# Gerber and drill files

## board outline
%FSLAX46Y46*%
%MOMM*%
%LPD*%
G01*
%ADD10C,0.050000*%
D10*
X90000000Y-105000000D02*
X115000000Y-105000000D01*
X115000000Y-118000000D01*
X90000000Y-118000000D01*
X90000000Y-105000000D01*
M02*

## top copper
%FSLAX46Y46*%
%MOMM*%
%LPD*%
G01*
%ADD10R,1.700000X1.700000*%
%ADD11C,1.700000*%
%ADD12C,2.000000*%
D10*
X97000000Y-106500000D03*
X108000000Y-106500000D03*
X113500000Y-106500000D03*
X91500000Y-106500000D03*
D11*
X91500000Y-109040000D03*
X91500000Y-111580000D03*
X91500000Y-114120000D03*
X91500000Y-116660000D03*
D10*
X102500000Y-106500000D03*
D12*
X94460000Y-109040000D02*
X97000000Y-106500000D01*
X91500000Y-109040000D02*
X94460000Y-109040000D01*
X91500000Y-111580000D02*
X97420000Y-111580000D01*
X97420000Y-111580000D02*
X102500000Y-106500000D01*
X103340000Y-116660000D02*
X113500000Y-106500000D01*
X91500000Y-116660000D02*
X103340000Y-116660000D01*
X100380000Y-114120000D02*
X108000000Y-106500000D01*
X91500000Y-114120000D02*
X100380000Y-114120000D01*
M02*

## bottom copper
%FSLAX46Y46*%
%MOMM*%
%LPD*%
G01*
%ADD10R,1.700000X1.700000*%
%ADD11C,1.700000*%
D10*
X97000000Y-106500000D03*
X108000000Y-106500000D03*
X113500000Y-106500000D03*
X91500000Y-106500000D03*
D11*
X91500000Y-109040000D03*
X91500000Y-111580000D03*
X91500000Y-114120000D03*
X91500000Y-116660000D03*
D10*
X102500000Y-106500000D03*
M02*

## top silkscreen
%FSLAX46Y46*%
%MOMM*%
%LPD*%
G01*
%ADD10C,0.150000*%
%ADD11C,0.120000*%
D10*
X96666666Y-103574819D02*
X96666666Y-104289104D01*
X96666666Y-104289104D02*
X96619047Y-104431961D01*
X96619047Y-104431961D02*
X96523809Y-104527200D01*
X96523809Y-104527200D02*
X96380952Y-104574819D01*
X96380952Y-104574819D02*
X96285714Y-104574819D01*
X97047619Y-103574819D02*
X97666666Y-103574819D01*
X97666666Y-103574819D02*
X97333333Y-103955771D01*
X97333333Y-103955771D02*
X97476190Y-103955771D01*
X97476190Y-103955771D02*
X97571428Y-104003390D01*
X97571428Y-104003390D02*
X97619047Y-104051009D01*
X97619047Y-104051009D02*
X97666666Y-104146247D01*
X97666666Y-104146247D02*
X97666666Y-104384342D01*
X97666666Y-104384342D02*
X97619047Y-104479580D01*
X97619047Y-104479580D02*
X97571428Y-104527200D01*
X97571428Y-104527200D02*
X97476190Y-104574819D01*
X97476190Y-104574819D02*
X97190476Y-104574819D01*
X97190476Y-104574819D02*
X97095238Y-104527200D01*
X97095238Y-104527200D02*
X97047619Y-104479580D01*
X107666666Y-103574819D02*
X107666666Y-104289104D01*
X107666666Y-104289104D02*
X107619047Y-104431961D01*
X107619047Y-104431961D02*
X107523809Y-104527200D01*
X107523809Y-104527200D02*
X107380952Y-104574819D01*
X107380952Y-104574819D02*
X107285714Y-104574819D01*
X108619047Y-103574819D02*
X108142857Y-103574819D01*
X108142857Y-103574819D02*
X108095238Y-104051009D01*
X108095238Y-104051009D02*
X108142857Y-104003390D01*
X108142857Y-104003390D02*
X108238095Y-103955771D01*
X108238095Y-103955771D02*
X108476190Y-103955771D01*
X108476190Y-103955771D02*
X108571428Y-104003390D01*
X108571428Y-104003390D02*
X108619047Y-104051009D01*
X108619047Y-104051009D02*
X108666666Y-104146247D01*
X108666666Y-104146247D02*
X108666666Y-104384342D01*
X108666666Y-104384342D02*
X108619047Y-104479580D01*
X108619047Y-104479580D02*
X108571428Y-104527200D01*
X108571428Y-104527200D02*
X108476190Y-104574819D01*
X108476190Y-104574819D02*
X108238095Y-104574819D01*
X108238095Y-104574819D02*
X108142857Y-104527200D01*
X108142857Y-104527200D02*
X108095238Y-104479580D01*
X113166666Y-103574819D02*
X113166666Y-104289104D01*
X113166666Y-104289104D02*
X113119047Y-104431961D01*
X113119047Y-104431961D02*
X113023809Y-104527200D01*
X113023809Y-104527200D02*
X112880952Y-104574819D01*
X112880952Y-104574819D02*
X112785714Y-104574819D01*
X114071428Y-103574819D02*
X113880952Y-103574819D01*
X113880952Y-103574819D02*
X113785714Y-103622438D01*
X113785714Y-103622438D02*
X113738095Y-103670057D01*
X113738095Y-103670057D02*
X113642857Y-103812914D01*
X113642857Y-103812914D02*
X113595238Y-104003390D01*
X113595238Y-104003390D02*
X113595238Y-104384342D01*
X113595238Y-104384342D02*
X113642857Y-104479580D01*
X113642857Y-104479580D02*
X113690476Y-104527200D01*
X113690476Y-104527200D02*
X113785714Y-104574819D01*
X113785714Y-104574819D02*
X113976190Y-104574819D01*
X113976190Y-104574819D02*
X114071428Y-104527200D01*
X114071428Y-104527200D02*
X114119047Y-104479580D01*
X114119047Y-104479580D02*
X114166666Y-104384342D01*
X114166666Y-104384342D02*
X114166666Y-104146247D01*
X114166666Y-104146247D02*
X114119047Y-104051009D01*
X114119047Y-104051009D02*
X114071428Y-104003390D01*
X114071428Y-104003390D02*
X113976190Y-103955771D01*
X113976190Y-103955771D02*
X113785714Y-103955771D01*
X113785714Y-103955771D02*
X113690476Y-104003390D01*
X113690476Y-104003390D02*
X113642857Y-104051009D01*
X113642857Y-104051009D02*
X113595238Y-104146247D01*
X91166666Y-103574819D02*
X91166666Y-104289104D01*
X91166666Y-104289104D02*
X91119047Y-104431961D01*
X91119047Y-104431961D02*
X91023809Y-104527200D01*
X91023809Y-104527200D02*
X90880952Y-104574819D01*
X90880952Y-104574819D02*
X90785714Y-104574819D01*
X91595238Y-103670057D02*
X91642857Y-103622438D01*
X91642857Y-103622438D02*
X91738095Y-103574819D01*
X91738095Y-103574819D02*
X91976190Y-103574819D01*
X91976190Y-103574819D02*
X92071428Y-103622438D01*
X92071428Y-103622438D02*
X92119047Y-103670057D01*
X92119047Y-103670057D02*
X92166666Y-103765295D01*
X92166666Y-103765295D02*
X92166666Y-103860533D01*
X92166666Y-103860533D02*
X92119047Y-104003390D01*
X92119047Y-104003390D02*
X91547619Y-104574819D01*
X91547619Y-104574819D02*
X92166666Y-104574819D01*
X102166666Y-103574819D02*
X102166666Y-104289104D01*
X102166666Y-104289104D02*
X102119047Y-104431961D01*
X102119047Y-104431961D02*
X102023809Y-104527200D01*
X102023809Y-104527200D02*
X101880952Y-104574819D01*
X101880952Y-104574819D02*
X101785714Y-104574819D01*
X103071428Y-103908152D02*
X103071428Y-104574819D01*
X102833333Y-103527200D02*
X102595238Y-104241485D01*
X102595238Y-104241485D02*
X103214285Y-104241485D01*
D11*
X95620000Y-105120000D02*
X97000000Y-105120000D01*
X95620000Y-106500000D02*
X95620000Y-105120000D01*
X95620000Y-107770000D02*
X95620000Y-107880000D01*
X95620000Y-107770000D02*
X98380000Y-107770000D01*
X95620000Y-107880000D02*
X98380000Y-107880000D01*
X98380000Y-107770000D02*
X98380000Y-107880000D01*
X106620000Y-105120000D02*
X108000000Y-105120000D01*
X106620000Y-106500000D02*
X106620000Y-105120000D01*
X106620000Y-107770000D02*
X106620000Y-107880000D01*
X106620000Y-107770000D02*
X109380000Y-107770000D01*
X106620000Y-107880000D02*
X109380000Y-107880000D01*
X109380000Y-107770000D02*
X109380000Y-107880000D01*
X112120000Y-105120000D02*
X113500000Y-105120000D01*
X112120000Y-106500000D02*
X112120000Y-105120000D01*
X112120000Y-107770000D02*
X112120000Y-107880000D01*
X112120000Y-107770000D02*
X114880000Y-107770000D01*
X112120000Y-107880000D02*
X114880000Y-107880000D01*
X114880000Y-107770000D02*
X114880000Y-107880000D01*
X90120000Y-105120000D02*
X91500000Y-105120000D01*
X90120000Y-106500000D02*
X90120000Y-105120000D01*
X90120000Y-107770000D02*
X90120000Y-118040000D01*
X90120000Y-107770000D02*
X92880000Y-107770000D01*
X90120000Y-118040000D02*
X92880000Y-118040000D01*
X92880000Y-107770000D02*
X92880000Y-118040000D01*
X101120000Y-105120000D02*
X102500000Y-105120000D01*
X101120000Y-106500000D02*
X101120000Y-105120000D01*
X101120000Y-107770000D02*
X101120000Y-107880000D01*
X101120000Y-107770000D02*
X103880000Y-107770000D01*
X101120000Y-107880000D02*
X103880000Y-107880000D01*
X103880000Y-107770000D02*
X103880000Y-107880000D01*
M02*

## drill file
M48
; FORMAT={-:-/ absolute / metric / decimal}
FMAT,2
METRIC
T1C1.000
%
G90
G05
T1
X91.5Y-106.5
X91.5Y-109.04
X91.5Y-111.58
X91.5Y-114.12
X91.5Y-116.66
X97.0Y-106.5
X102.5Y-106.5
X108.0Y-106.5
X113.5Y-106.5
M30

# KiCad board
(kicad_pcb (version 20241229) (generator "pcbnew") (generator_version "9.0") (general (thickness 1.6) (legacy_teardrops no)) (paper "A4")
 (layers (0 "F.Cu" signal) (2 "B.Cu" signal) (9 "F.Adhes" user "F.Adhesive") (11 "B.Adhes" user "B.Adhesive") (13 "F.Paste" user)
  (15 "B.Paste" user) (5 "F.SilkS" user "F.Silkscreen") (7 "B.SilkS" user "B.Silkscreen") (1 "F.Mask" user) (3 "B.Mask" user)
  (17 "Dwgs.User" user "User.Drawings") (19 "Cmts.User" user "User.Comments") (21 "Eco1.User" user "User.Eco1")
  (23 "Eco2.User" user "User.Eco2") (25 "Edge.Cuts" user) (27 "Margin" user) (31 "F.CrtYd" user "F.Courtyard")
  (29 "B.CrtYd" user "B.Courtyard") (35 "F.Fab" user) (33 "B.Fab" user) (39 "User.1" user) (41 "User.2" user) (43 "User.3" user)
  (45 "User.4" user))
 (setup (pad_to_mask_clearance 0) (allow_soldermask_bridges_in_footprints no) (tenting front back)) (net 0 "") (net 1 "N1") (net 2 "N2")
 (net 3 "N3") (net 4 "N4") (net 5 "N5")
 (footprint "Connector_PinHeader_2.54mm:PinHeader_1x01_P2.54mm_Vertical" (layer "F.Cu") (at 97 106.5)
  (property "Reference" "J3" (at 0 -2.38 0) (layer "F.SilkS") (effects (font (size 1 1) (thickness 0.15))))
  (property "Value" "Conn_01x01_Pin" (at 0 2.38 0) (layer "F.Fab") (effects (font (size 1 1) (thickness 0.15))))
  (fp_line (start -1.38 -1.38) (end 0 -1.38) (stroke (width 0.12) (type solid)) (layer "F.SilkS"))
  (fp_line (start -1.38 0) (end -1.38 -1.38) (stroke (width 0.12) (type solid)) (layer "F.SilkS"))
  (fp_line (start -1.38 1.27) (end -1.38 1.38) (stroke (width 0.12) (type solid)) (layer "F.SilkS"))
  (fp_line (start -1.38 1.27) (end 1.38 1.27) (stroke (width 0.12) (type solid)) (layer "F.SilkS"))
  (fp_line (start -1.38 1.38) (end 1.38 1.38) (stroke (width 0.12) (type solid)) (layer "F.SilkS"))
  (fp_line (start 1.38 1.27) (end 1.38 1.38) (stroke (width 0.12) (type solid)) (layer "F.SilkS"))
  (pad "1" thru_hole rect (at 0 0) (size 1.7 1.7) (drill 1) (layers "*.Cu" "*.Mask") (remove_unused_layers no) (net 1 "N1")))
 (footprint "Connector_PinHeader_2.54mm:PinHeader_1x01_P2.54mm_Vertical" (layer "F.Cu") (at 108 106.5)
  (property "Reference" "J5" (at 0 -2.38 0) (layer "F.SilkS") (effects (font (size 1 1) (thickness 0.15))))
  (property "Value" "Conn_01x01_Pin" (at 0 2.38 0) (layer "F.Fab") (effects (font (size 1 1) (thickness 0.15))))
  (fp_line (start -1.38 -1.38) (end 0 -1.38) (stroke (width 0.12) (type solid)) (layer "F.SilkS"))
  (fp_line (start -1.38 0) (end -1.38 -1.38) (stroke (width 0.12) (type solid)) (layer "F.SilkS"))
  (fp_line (start -1.38 1.27) (end -1.38 1.38) (stroke (width 0.12) (type solid)) (layer "F.SilkS"))
  (fp_line (start -1.38 1.27) (end 1.38 1.27) (stroke (width 0.12) (type solid)) (layer "F.SilkS"))
  (fp_line (start -1.38 1.38) (end 1.38 1.38) (stroke (width 0.12) (type solid)) (layer "F.SilkS"))
  (fp_line (start 1.38 1.27) (end 1.38 1.38) (stroke (width 0.12) (type solid)) (layer "F.SilkS"))
  (pad "1" thru_hole rect (at 0 0) (size 1.7 1.7) (drill 1) (layers "*.Cu" "*.Mask") (remove_unused_layers no) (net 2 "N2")))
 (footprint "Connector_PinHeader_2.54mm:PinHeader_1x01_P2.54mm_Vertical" (layer "F.Cu") (at 113.5 106.5)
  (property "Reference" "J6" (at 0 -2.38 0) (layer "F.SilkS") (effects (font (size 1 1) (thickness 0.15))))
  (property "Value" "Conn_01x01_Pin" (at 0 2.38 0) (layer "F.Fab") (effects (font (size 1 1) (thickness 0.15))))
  (fp_line (start -1.38 -1.38) (end 0 -1.38) (stroke (width 0.12) (type solid)) (layer "F.SilkS"))
  (fp_line (start -1.38 0) (end -1.38 -1.38) (stroke (width 0.12) (type solid)) (layer "F.SilkS"))
  (fp_line (start -1.38 1.27) (end -1.38 1.38) (stroke (width 0.12) (type solid)) (layer "F.SilkS"))
  (fp_line (start -1.38 1.27) (end 1.38 1.27) (stroke (width 0.12) (type solid)) (layer "F.SilkS"))
  (fp_line (start -1.38 1.38) (end 1.38 1.38) (stroke (width 0.12) (type solid)) (layer "F.SilkS"))
  (fp_line (start 1.38 1.27) (end 1.38 1.38) (stroke (width 0.12) (type solid)) (layer "F.SilkS"))
  (pad "1" thru_hole rect (at 0 0) (size 1.7 1.7) (drill 1) (layers "*.Cu" "*.Mask") (remove_unused_layers no) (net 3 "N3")))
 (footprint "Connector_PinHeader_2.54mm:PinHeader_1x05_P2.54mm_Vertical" (layer "F.Cu") (at 91.5 106.5)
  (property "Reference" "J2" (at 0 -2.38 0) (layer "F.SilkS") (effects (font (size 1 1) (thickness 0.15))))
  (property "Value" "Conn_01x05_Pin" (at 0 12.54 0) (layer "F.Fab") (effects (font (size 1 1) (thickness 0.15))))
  (fp_line (start -1.38 -1.38) (end 0 -1.38) (stroke (width 0.12) (type solid)) (layer "F.SilkS"))
  (fp_line (start -1.38 0) (end -1.38 -1.38) (stroke (width 0.12) (type solid)) (layer "F.SilkS"))
  (fp_line (start -1.38 1.27) (end -1.38 11.54) (stroke (width 0.12) (type solid)) (layer "F.SilkS"))
  (fp_line (start -1.38 1.27) (end 1.38 1.27) (stroke (width 0.12) (type solid)) (layer "F.SilkS"))
  (fp_line (start -1.38 11.54) (end 1.38 11.54) (stroke (width 0.12) (type solid)) (layer "F.SilkS"))
  (fp_line (start 1.38 1.27) (end 1.38 11.54) (stroke (width 0.12) (type solid)) (layer "F.SilkS"))
  (pad "1" thru_hole rect (at 0 0) (size 1.7 1.7) (drill 1) (layers "*.Cu" "*.Mask") (remove_unused_layers no) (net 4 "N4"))
  (pad "2" thru_hole circle (at 0 2.54) (size 1.7 1.7) (drill 1) (layers "*.Cu" "*.Mask") (remove_unused_layers no) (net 1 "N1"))
  (pad "3" thru_hole circle (at 0 5.08) (size 1.7 1.7) (drill 1) (layers "*.Cu" "*.Mask") (remove_unused_layers no) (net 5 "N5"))
  (pad "4" thru_hole circle (at 0 7.62) (size 1.7 1.7) (drill 1) (layers "*.Cu" "*.Mask") (remove_unused_layers no) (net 2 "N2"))
  (pad "5" thru_hole circle (at 0 10.16) (size 1.7 1.7) (drill 1) (layers "*.Cu" "*.Mask") (remove_unused_layers no) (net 3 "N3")))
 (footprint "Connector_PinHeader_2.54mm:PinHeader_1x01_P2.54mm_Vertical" (layer "F.Cu") (at 102.5 106.5)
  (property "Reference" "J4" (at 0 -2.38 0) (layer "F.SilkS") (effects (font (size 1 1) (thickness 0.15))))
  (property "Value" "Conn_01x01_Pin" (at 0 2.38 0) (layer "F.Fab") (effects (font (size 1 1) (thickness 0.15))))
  (fp_line (start -1.38 -1.38) (end 0 -1.38) (stroke (width 0.12) (type solid)) (layer "F.SilkS"))
  (fp_line (start -1.38 0) (end -1.38 -1.38) (stroke (width 0.12) (type solid)) (layer "F.SilkS"))
  (fp_line (start -1.38 1.27) (end -1.38 1.38) (stroke (width 0.12) (type solid)) (layer "F.SilkS"))
  (fp_line (start -1.38 1.27) (end 1.38 1.27) (stroke (width 0.12) (type solid)) (layer "F.SilkS"))
  (fp_line (start -1.38 1.38) (end 1.38 1.38) (stroke (width 0.12) (type solid)) (layer "F.SilkS"))
  (fp_line (start 1.38 1.27) (end 1.38 1.38) (stroke (width 0.12) (type solid)) (layer "F.SilkS"))
  (pad "1" thru_hole rect (at 0 0) (size 1.7 1.7) (drill 1) (layers "*.Cu" "*.Mask") (remove_unused_layers no) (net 5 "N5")))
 (gr_rect (start 90 105) (end 115 118) (stroke (width 0.05) (type default)) (fill no) (layer "Edge.Cuts"))
 (segment (start 94.46 109.04) (end 97 106.5) (width 2) (layer "F.Cu") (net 1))
 (segment (start 91.5 109.04) (end 94.46 109.04) (width 2) (layer "F.Cu") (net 1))
 (segment (start 91.5 111.58) (end 97.42 111.58) (width 2) (layer "F.Cu") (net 5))
 (segment (start 97.42 111.58) (end 102.5 106.5) (width 2) (layer "F.Cu") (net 5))
 (segment (start 103.34 116.66) (end 113.5 106.5) (width 2) (layer "F.Cu") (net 3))
 (segment (start 91.5 116.66) (end 103.34 116.66) (width 2) (layer "F.Cu") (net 3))
 (segment (start 100.38 114.12) (end 108 106.5) (width 2) (layer "F.Cu") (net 2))
 (segment (start 91.5 114.12) (end 100.38 114.12) (width 2) (layer "F.Cu") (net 2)))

